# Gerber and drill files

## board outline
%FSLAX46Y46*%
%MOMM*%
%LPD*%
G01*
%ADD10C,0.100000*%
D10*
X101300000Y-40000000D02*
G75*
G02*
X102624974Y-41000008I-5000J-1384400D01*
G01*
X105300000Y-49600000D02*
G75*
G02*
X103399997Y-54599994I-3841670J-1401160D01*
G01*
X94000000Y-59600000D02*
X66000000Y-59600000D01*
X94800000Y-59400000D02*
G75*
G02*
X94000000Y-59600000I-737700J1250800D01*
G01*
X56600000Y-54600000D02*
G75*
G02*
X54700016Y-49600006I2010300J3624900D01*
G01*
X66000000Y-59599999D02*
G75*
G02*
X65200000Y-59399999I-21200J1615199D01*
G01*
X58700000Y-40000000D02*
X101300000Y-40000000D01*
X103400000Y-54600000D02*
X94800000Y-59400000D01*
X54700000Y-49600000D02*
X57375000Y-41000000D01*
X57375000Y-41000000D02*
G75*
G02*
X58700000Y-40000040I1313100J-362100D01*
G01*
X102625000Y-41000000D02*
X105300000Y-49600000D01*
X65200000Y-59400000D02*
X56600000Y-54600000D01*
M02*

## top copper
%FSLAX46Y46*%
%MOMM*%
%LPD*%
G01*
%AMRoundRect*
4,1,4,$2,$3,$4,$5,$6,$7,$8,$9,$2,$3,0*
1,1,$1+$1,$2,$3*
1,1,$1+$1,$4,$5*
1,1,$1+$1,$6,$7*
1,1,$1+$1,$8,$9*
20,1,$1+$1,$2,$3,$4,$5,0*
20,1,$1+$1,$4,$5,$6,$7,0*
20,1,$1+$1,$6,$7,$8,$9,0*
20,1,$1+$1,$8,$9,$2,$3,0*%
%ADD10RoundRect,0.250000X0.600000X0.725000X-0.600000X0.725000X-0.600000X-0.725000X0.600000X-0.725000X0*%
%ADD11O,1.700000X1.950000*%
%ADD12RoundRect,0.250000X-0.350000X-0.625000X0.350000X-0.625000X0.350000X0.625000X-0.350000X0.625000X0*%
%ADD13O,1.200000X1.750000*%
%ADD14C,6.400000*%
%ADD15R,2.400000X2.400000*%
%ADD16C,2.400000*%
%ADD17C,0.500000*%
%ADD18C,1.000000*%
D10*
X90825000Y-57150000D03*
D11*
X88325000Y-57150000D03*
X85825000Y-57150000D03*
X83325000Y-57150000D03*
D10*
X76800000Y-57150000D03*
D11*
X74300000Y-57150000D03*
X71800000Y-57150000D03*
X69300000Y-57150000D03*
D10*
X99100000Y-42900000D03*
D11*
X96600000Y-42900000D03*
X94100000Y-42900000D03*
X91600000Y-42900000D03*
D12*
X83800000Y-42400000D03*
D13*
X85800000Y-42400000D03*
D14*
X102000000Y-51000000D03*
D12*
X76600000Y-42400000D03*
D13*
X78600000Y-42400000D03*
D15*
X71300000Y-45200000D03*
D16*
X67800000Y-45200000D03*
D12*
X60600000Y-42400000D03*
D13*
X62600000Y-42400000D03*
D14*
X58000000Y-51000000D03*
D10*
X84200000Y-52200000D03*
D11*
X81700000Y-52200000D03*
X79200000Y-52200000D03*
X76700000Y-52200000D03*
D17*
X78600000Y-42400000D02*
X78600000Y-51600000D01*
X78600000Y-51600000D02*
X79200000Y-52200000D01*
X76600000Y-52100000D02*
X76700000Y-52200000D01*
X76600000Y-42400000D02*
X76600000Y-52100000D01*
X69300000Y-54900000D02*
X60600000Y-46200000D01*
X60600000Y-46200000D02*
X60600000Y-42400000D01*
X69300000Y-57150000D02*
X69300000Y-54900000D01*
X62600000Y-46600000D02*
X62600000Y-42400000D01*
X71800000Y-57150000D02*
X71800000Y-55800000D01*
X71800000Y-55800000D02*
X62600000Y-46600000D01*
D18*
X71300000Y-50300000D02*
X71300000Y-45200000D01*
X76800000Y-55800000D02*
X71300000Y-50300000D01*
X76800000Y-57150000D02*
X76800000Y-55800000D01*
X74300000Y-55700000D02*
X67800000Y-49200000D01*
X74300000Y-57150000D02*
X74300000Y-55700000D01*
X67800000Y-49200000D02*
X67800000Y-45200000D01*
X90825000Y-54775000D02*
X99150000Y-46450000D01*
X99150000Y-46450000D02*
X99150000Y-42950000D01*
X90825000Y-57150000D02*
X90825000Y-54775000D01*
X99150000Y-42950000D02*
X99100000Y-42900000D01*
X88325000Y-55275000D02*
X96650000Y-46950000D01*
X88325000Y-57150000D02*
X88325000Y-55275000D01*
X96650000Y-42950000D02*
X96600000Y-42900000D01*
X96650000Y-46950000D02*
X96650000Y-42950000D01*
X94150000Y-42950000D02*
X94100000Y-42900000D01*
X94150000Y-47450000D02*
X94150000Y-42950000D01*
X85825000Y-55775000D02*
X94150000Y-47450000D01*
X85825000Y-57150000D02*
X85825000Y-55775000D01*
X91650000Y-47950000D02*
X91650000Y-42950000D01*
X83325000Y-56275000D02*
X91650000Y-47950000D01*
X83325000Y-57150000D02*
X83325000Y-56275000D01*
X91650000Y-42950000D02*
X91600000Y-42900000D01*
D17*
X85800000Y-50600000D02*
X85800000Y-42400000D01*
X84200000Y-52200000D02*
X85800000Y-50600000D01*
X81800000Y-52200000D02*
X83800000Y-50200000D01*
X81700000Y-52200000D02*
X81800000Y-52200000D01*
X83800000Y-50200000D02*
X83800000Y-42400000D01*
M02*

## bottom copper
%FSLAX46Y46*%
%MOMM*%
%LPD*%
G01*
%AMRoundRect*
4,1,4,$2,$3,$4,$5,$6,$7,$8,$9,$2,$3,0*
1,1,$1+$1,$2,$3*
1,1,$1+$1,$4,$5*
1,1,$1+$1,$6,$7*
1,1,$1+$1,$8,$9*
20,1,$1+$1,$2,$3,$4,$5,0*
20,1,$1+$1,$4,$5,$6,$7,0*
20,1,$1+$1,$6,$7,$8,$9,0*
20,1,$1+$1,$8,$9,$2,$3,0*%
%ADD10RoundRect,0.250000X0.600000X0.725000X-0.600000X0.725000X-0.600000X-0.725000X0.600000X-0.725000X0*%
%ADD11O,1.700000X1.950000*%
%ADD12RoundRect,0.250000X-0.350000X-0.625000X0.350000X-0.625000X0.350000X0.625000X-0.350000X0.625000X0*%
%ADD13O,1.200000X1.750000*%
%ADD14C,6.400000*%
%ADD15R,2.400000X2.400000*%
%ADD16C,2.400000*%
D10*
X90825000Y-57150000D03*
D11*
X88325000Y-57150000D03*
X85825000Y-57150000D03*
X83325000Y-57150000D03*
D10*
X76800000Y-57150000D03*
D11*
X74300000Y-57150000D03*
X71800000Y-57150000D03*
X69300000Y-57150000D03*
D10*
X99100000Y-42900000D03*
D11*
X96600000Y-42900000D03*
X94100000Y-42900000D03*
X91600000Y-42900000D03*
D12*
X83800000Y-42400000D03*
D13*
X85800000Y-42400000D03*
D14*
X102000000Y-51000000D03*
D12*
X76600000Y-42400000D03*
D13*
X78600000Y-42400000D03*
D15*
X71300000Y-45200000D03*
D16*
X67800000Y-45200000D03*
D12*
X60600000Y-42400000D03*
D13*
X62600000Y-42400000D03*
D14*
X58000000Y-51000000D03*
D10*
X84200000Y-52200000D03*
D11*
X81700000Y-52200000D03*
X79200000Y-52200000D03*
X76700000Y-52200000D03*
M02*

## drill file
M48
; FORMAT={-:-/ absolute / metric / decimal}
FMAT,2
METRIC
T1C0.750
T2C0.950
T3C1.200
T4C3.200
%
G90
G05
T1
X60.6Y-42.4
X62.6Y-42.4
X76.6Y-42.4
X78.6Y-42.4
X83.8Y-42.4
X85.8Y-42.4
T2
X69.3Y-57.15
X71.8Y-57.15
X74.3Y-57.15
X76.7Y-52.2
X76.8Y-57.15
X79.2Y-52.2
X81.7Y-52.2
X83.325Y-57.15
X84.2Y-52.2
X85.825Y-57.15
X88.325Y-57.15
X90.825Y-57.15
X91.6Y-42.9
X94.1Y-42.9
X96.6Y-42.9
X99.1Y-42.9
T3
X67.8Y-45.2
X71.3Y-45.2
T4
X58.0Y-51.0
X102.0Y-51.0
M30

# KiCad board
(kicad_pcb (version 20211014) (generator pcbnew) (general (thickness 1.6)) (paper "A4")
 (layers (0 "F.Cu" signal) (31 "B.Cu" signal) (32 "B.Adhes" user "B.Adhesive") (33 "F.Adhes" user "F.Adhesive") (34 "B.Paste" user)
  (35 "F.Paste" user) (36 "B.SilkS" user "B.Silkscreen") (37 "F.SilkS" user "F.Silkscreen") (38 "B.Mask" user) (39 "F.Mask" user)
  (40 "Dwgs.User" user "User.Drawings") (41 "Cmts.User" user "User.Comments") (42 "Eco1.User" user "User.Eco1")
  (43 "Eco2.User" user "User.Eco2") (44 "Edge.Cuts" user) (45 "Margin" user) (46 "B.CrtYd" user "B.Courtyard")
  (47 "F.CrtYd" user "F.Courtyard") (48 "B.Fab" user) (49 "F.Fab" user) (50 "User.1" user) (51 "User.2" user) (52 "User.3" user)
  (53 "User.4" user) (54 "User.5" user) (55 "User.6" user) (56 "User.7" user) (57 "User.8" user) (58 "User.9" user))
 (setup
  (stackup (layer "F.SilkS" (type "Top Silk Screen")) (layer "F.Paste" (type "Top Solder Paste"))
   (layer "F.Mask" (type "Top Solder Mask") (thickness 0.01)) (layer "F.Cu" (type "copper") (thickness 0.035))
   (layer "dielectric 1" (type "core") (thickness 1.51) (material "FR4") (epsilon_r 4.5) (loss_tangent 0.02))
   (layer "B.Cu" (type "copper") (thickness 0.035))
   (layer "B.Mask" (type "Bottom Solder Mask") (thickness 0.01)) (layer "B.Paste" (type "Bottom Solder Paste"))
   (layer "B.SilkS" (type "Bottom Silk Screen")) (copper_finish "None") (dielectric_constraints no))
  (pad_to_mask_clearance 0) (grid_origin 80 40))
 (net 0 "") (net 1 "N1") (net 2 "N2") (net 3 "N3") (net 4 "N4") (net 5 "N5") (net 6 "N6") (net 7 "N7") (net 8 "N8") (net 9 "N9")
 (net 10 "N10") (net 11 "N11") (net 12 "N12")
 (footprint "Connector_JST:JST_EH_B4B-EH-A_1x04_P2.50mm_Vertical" (layer "F.Cu") (at 90.825 57.15 180)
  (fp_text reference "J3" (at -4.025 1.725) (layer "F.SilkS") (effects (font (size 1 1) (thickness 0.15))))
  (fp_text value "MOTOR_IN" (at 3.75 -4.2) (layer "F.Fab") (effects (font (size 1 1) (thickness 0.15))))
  (pad "1" thru_hole roundrect (at 0 0 180) (size 1.7 1.95) (drill 0.95) (layers *.Cu *.Mask) (roundrect_rratio 0.147059) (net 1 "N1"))
  (pad "2" thru_hole oval (at 2.5 0 180) (size 1.7 1.95) (drill 0.95) (layers *.Cu *.Mask) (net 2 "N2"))
  (pad "3" thru_hole oval (at 5 0 180) (size 1.7 1.95) (drill 0.95) (layers *.Cu *.Mask) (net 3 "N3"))
  (pad "4" thru_hole oval (at 7.5 0 180) (size 1.7 1.95) (drill 0.95) (layers *.Cu *.Mask) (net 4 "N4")))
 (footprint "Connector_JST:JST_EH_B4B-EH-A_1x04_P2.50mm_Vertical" (layer "F.Cu") (at 76.8 57.15 180)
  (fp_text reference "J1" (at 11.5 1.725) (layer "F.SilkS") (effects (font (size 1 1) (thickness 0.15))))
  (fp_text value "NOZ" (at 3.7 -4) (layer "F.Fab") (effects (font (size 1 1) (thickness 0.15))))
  (pad "1" thru_hole roundrect (at 0 0 180) (size 1.7 1.95) (drill 0.95) (layers *.Cu *.Mask) (roundrect_rratio 0.147059) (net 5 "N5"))
  (pad "2" thru_hole oval (at 2.5 0 180) (size 1.7 1.95) (drill 0.95) (layers *.Cu *.Mask) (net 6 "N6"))
  (pad "3" thru_hole oval (at 5 0 180) (size 1.7 1.95) (drill 0.95) (layers *.Cu *.Mask) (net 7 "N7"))
  (pad "4" thru_hole oval (at 7.5 0 180) (size 1.7 1.95) (drill 0.95) (layers *.Cu *.Mask) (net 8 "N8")))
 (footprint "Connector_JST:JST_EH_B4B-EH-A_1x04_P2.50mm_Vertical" (layer "F.Cu") (at 99.1 42.9 180)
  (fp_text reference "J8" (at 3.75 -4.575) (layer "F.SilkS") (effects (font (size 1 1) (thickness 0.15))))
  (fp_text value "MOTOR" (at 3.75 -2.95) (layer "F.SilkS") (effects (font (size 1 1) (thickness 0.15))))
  (pad "1" thru_hole roundrect (at 0 0 180) (size 1.7 1.95) (drill 0.95) (layers *.Cu *.Mask) (roundrect_rratio 0.147059) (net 1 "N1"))
  (pad "2" thru_hole oval (at 2.5 0 180) (size 1.7 1.95) (drill 0.95) (layers *.Cu *.Mask) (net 2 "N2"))
  (pad "3" thru_hole oval (at 5 0 180) (size 1.7 1.95) (drill 0.95) (layers *.Cu *.Mask) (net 3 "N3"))
  (pad "4" thru_hole oval (at 7.5 0 180) (size 1.7 1.95) (drill 0.95) (layers *.Cu *.Mask) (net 4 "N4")))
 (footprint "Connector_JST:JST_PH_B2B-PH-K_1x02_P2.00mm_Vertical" (layer "F.Cu") (at 83.8 42.4)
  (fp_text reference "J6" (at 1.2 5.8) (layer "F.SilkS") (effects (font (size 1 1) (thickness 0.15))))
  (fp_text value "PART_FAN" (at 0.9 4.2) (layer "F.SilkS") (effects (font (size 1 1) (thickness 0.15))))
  (pad "1" thru_hole roundrect (at 0 0) (size 1.2 1.75) (drill 0.75) (layers *.Cu *.Mask) (roundrect_rratio 0.208333) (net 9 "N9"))
  (pad "2" thru_hole oval (at 2 0) (size 1.2 1.75) (drill 0.75) (layers *.Cu *.Mask) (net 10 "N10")))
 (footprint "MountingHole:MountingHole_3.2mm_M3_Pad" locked (layer "F.Cu") (at 102 51)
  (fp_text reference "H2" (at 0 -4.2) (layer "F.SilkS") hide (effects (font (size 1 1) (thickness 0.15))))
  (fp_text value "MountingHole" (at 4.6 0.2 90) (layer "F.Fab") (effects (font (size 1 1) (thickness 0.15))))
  (pad "1" thru_hole circle locked (at 0 0) (size 6.4 6.4) (drill 3.2) (layers *.Cu *.Mask)))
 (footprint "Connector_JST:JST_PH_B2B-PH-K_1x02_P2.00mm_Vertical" (layer "F.Cu") (at 76.6 42.4)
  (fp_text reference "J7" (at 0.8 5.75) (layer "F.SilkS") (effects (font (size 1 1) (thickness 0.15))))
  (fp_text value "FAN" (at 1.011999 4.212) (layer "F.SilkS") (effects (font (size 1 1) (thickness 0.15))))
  (pad "1" thru_hole roundrect (at 0 0) (size 1.2 1.75) (drill 0.75) (layers *.Cu *.Mask) (roundrect_rratio 0.208333) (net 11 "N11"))
  (pad "2" thru_hole oval (at 2 0) (size 1.2 1.75) (drill 0.75) (layers *.Cu *.Mask) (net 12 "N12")))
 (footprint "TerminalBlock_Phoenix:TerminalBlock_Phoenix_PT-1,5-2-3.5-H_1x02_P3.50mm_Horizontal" (layer "F.Cu") (at 71.3 45.2 180)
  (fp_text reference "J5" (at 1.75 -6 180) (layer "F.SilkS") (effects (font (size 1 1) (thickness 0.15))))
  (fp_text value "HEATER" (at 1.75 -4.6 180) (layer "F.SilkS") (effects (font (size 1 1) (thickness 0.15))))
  (pad "1" thru_hole rect (at 0 0 180) (size 2.4 2.4) (drill 1.2) (layers *.Cu *.Mask) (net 5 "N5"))
  (pad "2" thru_hole circle (at 3.5 0 180) (size 2.4 2.4) (drill 1.2) (layers *.Cu *.Mask) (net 6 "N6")))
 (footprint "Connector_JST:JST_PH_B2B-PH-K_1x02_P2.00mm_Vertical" (layer "F.Cu") (at 60.6 42.4)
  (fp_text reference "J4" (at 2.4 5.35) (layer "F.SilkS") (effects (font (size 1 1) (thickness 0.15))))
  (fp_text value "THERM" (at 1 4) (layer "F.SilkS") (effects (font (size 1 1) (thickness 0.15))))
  (pad "1" thru_hole roundrect (at 0 0) (size 1.2 1.75) (drill 0.75) (layers *.Cu *.Mask) (roundrect_rratio 0.208333) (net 8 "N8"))
  (pad "2" thru_hole oval (at 2 0) (size 1.2 1.75) (drill 0.75) (layers *.Cu *.Mask) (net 7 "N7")))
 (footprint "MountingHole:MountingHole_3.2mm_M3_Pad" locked (layer "F.Cu") (at 58 51)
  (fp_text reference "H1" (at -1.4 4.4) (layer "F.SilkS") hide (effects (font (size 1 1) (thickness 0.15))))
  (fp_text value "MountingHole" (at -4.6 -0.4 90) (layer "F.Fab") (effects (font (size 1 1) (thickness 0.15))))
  (pad "1" thru_hole circle locked (at 0 0) (size 6.4 6.4) (drill 3.2) (layers *.Cu *.Mask)))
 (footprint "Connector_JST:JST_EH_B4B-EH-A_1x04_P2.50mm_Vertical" (layer "F.Cu") (at 84.2 52.2 180)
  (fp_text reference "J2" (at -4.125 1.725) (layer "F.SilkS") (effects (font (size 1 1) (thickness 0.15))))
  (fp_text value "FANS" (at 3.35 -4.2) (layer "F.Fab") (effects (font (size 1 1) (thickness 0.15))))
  (pad "1" thru_hole roundrect (at 0 0 180) (size 1.7 1.95) (drill 0.95) (layers *.Cu *.Mask) (roundrect_rratio 0.147059) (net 10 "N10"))
  (pad "2" thru_hole oval (at 2.5 0 180) (size 1.7 1.95) (drill 0.95) (layers *.Cu *.Mask) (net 9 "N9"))
  (pad "3" thru_hole oval (at 5 0 180) (size 1.7 1.95) (drill 0.95) (layers *.Cu *.Mask) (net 12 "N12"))
  (pad "4" thru_hole oval (at 7.5 0 180) (size 1.7 1.95) (drill 0.95) (layers *.Cu *.Mask) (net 11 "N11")))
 (gr_arc (start 101.3 40) (mid 102.129008 40.27938) (end 102.625 41) (layer "Edge.Cuts") (width 0.1))
 (gr_arc (start 105.3 49.6) (mid 105.280862 52.453728) (end 103.4 54.6) (layer "Edge.Cuts") (width 0.1))
 (gr_line (start 94 59.6) (end 66 59.6) (layer "Edge.Cuts") (width 0.1))
 (gr_arc (start 94.8 59.4) (mid 94.414494 59.557982) (end 94 59.6) (layer "Edge.Cuts") (width 0.1))
 (gr_arc (start 56.6 54.6) (mid 54.735582 52.447479) (end 54.7 49.6) (layer "Edge.Cuts") (width 0.1))
 (gr_arc (start 66 59.599999) (mid 65.587022 59.55191) (end 65.2 59.4) (layer "Edge.Cuts") (width 0.1))
 (gr_line (start 58.7 40) (end 101.3 40) (layer "Edge.Cuts") (width 0.1))
 (gr_line (start 103.4 54.6) (end 94.8 59.4) (layer "Edge.Cuts") (width 0.1))
 (gr_line (start 54.7 49.6) (end 57.375 41) (layer "Edge.Cuts") (width 0.1))
 (gr_arc (start 57.375 41) (mid 57.867573 40.274847) (end 58.7 40) (layer "Edge.Cuts") (width 0.1))
 (gr_line (start 102.625 41) (end 105.3 49.6) (layer "Edge.Cuts") (width 0.1))
 (gr_line (start 65.2 59.4) (end 56.6 54.6) (layer "Edge.Cuts") (width 0.1))
 (segment (start 78.6 42.4) (end 78.6 51.6) (width 0.5) (layer "F.Cu") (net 12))
 (segment (start 78.6 51.6) (end 79.2 52.2) (width 0.5) (layer "F.Cu") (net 12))
 (segment (start 76.6 52.1) (end 76.7 52.2) (width 0.5) (layer "F.Cu") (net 11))
 (segment (start 76.6 42.4) (end 76.6 52.1) (width 0.5) (layer "F.Cu") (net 11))
 (segment (start 69.3 54.9) (end 60.6 46.2) (width 0.5) (layer "F.Cu") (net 8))
 (segment (start 60.6 46.2) (end 60.6 42.4) (width 0.5) (layer "F.Cu") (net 8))
 (segment (start 69.3 57.15) (end 69.3 54.9) (width 0.5) (layer "F.Cu") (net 8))
 (segment (start 62.6 46.6) (end 62.6 42.4) (width 0.5) (layer "F.Cu") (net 7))
 (segment (start 71.8 57.15) (end 71.8 55.8) (width 0.5) (layer "F.Cu") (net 7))
 (segment (start 71.8 55.8) (end 62.6 46.6) (width 0.5) (layer "F.Cu") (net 7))
 (segment (start 71.3 50.3) (end 71.3 45.2) (width 1) (layer "F.Cu") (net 5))
 (segment (start 76.8 55.8) (end 71.3 50.3) (width 1) (layer "F.Cu") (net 5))
 (segment (start 76.8 57.15) (end 76.8 55.8) (width 1) (layer "F.Cu") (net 5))
 (segment (start 74.3 55.7) (end 67.8 49.2) (width 1) (layer "F.Cu") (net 6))
 (segment (start 74.3 57.15) (end 74.3 55.7) (width 1) (layer "F.Cu") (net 6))
 (segment (start 67.8 49.2) (end 67.8 45.2) (width 1) (layer "F.Cu") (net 6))
 (segment (start 90.825 54.775) (end 99.15 46.45) (width 1) (layer "F.Cu") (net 1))
 (segment (start 99.15 46.45) (end 99.15 42.95) (width 1) (layer "F.Cu") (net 1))
 (segment (start 90.825 57.15) (end 90.825 54.775) (width 1) (layer "F.Cu") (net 1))
 (segment (start 99.15 42.95) (end 99.1 42.9) (width 1) (layer "F.Cu") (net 1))
 (segment (start 88.325 55.275) (end 96.65 46.95) (width 1) (layer "F.Cu") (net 2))
 (segment (start 88.325 57.15) (end 88.325 55.275) (width 1) (layer "F.Cu") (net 2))
 (segment (start 96.65 42.95) (end 96.6 42.9) (width 1) (layer "F.Cu") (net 2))
 (segment (start 96.65 46.95) (end 96.65 42.95) (width 1) (layer "F.Cu") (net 2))
 (segment (start 94.15 42.95) (end 94.1 42.9) (width 1) (layer "F.Cu") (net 3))
 (segment (start 94.15 47.45) (end 94.15 42.95) (width 1) (layer "F.Cu") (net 3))
 (segment (start 85.825 55.775) (end 94.15 47.45) (width 1) (layer "F.Cu") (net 3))
 (segment (start 85.825 57.15) (end 85.825 55.775) (width 1) (layer "F.Cu") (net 3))
 (segment (start 91.65 47.95) (end 91.65 42.95) (width 1) (layer "F.Cu") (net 4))
 (segment (start 83.325 56.275) (end 91.65 47.95) (width 1) (layer "F.Cu") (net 4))
 (segment (start 83.325 57.15) (end 83.325 56.275) (width 1) (layer "F.Cu") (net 4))
 (segment (start 91.65 42.95) (end 91.6 42.9) (width 1) (layer "F.Cu") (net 4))
 (segment (start 85.8 50.6) (end 85.8 42.4) (width 0.5) (layer "F.Cu") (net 10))
 (segment (start 84.2 52.2) (end 85.8 50.6) (width 0.5) (layer "F.Cu") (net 10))
 (segment (start 81.8 52.2) (end 83.8 50.2) (width 0.5) (layer "F.Cu") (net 9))
 (segment (start 81.7 52.2) (end 81.8 52.2) (width 0.5) (layer "F.Cu") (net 9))
 (segment (start 83.8 50.2) (end 83.8 42.4) (width 0.5) (layer "F.Cu") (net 9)))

